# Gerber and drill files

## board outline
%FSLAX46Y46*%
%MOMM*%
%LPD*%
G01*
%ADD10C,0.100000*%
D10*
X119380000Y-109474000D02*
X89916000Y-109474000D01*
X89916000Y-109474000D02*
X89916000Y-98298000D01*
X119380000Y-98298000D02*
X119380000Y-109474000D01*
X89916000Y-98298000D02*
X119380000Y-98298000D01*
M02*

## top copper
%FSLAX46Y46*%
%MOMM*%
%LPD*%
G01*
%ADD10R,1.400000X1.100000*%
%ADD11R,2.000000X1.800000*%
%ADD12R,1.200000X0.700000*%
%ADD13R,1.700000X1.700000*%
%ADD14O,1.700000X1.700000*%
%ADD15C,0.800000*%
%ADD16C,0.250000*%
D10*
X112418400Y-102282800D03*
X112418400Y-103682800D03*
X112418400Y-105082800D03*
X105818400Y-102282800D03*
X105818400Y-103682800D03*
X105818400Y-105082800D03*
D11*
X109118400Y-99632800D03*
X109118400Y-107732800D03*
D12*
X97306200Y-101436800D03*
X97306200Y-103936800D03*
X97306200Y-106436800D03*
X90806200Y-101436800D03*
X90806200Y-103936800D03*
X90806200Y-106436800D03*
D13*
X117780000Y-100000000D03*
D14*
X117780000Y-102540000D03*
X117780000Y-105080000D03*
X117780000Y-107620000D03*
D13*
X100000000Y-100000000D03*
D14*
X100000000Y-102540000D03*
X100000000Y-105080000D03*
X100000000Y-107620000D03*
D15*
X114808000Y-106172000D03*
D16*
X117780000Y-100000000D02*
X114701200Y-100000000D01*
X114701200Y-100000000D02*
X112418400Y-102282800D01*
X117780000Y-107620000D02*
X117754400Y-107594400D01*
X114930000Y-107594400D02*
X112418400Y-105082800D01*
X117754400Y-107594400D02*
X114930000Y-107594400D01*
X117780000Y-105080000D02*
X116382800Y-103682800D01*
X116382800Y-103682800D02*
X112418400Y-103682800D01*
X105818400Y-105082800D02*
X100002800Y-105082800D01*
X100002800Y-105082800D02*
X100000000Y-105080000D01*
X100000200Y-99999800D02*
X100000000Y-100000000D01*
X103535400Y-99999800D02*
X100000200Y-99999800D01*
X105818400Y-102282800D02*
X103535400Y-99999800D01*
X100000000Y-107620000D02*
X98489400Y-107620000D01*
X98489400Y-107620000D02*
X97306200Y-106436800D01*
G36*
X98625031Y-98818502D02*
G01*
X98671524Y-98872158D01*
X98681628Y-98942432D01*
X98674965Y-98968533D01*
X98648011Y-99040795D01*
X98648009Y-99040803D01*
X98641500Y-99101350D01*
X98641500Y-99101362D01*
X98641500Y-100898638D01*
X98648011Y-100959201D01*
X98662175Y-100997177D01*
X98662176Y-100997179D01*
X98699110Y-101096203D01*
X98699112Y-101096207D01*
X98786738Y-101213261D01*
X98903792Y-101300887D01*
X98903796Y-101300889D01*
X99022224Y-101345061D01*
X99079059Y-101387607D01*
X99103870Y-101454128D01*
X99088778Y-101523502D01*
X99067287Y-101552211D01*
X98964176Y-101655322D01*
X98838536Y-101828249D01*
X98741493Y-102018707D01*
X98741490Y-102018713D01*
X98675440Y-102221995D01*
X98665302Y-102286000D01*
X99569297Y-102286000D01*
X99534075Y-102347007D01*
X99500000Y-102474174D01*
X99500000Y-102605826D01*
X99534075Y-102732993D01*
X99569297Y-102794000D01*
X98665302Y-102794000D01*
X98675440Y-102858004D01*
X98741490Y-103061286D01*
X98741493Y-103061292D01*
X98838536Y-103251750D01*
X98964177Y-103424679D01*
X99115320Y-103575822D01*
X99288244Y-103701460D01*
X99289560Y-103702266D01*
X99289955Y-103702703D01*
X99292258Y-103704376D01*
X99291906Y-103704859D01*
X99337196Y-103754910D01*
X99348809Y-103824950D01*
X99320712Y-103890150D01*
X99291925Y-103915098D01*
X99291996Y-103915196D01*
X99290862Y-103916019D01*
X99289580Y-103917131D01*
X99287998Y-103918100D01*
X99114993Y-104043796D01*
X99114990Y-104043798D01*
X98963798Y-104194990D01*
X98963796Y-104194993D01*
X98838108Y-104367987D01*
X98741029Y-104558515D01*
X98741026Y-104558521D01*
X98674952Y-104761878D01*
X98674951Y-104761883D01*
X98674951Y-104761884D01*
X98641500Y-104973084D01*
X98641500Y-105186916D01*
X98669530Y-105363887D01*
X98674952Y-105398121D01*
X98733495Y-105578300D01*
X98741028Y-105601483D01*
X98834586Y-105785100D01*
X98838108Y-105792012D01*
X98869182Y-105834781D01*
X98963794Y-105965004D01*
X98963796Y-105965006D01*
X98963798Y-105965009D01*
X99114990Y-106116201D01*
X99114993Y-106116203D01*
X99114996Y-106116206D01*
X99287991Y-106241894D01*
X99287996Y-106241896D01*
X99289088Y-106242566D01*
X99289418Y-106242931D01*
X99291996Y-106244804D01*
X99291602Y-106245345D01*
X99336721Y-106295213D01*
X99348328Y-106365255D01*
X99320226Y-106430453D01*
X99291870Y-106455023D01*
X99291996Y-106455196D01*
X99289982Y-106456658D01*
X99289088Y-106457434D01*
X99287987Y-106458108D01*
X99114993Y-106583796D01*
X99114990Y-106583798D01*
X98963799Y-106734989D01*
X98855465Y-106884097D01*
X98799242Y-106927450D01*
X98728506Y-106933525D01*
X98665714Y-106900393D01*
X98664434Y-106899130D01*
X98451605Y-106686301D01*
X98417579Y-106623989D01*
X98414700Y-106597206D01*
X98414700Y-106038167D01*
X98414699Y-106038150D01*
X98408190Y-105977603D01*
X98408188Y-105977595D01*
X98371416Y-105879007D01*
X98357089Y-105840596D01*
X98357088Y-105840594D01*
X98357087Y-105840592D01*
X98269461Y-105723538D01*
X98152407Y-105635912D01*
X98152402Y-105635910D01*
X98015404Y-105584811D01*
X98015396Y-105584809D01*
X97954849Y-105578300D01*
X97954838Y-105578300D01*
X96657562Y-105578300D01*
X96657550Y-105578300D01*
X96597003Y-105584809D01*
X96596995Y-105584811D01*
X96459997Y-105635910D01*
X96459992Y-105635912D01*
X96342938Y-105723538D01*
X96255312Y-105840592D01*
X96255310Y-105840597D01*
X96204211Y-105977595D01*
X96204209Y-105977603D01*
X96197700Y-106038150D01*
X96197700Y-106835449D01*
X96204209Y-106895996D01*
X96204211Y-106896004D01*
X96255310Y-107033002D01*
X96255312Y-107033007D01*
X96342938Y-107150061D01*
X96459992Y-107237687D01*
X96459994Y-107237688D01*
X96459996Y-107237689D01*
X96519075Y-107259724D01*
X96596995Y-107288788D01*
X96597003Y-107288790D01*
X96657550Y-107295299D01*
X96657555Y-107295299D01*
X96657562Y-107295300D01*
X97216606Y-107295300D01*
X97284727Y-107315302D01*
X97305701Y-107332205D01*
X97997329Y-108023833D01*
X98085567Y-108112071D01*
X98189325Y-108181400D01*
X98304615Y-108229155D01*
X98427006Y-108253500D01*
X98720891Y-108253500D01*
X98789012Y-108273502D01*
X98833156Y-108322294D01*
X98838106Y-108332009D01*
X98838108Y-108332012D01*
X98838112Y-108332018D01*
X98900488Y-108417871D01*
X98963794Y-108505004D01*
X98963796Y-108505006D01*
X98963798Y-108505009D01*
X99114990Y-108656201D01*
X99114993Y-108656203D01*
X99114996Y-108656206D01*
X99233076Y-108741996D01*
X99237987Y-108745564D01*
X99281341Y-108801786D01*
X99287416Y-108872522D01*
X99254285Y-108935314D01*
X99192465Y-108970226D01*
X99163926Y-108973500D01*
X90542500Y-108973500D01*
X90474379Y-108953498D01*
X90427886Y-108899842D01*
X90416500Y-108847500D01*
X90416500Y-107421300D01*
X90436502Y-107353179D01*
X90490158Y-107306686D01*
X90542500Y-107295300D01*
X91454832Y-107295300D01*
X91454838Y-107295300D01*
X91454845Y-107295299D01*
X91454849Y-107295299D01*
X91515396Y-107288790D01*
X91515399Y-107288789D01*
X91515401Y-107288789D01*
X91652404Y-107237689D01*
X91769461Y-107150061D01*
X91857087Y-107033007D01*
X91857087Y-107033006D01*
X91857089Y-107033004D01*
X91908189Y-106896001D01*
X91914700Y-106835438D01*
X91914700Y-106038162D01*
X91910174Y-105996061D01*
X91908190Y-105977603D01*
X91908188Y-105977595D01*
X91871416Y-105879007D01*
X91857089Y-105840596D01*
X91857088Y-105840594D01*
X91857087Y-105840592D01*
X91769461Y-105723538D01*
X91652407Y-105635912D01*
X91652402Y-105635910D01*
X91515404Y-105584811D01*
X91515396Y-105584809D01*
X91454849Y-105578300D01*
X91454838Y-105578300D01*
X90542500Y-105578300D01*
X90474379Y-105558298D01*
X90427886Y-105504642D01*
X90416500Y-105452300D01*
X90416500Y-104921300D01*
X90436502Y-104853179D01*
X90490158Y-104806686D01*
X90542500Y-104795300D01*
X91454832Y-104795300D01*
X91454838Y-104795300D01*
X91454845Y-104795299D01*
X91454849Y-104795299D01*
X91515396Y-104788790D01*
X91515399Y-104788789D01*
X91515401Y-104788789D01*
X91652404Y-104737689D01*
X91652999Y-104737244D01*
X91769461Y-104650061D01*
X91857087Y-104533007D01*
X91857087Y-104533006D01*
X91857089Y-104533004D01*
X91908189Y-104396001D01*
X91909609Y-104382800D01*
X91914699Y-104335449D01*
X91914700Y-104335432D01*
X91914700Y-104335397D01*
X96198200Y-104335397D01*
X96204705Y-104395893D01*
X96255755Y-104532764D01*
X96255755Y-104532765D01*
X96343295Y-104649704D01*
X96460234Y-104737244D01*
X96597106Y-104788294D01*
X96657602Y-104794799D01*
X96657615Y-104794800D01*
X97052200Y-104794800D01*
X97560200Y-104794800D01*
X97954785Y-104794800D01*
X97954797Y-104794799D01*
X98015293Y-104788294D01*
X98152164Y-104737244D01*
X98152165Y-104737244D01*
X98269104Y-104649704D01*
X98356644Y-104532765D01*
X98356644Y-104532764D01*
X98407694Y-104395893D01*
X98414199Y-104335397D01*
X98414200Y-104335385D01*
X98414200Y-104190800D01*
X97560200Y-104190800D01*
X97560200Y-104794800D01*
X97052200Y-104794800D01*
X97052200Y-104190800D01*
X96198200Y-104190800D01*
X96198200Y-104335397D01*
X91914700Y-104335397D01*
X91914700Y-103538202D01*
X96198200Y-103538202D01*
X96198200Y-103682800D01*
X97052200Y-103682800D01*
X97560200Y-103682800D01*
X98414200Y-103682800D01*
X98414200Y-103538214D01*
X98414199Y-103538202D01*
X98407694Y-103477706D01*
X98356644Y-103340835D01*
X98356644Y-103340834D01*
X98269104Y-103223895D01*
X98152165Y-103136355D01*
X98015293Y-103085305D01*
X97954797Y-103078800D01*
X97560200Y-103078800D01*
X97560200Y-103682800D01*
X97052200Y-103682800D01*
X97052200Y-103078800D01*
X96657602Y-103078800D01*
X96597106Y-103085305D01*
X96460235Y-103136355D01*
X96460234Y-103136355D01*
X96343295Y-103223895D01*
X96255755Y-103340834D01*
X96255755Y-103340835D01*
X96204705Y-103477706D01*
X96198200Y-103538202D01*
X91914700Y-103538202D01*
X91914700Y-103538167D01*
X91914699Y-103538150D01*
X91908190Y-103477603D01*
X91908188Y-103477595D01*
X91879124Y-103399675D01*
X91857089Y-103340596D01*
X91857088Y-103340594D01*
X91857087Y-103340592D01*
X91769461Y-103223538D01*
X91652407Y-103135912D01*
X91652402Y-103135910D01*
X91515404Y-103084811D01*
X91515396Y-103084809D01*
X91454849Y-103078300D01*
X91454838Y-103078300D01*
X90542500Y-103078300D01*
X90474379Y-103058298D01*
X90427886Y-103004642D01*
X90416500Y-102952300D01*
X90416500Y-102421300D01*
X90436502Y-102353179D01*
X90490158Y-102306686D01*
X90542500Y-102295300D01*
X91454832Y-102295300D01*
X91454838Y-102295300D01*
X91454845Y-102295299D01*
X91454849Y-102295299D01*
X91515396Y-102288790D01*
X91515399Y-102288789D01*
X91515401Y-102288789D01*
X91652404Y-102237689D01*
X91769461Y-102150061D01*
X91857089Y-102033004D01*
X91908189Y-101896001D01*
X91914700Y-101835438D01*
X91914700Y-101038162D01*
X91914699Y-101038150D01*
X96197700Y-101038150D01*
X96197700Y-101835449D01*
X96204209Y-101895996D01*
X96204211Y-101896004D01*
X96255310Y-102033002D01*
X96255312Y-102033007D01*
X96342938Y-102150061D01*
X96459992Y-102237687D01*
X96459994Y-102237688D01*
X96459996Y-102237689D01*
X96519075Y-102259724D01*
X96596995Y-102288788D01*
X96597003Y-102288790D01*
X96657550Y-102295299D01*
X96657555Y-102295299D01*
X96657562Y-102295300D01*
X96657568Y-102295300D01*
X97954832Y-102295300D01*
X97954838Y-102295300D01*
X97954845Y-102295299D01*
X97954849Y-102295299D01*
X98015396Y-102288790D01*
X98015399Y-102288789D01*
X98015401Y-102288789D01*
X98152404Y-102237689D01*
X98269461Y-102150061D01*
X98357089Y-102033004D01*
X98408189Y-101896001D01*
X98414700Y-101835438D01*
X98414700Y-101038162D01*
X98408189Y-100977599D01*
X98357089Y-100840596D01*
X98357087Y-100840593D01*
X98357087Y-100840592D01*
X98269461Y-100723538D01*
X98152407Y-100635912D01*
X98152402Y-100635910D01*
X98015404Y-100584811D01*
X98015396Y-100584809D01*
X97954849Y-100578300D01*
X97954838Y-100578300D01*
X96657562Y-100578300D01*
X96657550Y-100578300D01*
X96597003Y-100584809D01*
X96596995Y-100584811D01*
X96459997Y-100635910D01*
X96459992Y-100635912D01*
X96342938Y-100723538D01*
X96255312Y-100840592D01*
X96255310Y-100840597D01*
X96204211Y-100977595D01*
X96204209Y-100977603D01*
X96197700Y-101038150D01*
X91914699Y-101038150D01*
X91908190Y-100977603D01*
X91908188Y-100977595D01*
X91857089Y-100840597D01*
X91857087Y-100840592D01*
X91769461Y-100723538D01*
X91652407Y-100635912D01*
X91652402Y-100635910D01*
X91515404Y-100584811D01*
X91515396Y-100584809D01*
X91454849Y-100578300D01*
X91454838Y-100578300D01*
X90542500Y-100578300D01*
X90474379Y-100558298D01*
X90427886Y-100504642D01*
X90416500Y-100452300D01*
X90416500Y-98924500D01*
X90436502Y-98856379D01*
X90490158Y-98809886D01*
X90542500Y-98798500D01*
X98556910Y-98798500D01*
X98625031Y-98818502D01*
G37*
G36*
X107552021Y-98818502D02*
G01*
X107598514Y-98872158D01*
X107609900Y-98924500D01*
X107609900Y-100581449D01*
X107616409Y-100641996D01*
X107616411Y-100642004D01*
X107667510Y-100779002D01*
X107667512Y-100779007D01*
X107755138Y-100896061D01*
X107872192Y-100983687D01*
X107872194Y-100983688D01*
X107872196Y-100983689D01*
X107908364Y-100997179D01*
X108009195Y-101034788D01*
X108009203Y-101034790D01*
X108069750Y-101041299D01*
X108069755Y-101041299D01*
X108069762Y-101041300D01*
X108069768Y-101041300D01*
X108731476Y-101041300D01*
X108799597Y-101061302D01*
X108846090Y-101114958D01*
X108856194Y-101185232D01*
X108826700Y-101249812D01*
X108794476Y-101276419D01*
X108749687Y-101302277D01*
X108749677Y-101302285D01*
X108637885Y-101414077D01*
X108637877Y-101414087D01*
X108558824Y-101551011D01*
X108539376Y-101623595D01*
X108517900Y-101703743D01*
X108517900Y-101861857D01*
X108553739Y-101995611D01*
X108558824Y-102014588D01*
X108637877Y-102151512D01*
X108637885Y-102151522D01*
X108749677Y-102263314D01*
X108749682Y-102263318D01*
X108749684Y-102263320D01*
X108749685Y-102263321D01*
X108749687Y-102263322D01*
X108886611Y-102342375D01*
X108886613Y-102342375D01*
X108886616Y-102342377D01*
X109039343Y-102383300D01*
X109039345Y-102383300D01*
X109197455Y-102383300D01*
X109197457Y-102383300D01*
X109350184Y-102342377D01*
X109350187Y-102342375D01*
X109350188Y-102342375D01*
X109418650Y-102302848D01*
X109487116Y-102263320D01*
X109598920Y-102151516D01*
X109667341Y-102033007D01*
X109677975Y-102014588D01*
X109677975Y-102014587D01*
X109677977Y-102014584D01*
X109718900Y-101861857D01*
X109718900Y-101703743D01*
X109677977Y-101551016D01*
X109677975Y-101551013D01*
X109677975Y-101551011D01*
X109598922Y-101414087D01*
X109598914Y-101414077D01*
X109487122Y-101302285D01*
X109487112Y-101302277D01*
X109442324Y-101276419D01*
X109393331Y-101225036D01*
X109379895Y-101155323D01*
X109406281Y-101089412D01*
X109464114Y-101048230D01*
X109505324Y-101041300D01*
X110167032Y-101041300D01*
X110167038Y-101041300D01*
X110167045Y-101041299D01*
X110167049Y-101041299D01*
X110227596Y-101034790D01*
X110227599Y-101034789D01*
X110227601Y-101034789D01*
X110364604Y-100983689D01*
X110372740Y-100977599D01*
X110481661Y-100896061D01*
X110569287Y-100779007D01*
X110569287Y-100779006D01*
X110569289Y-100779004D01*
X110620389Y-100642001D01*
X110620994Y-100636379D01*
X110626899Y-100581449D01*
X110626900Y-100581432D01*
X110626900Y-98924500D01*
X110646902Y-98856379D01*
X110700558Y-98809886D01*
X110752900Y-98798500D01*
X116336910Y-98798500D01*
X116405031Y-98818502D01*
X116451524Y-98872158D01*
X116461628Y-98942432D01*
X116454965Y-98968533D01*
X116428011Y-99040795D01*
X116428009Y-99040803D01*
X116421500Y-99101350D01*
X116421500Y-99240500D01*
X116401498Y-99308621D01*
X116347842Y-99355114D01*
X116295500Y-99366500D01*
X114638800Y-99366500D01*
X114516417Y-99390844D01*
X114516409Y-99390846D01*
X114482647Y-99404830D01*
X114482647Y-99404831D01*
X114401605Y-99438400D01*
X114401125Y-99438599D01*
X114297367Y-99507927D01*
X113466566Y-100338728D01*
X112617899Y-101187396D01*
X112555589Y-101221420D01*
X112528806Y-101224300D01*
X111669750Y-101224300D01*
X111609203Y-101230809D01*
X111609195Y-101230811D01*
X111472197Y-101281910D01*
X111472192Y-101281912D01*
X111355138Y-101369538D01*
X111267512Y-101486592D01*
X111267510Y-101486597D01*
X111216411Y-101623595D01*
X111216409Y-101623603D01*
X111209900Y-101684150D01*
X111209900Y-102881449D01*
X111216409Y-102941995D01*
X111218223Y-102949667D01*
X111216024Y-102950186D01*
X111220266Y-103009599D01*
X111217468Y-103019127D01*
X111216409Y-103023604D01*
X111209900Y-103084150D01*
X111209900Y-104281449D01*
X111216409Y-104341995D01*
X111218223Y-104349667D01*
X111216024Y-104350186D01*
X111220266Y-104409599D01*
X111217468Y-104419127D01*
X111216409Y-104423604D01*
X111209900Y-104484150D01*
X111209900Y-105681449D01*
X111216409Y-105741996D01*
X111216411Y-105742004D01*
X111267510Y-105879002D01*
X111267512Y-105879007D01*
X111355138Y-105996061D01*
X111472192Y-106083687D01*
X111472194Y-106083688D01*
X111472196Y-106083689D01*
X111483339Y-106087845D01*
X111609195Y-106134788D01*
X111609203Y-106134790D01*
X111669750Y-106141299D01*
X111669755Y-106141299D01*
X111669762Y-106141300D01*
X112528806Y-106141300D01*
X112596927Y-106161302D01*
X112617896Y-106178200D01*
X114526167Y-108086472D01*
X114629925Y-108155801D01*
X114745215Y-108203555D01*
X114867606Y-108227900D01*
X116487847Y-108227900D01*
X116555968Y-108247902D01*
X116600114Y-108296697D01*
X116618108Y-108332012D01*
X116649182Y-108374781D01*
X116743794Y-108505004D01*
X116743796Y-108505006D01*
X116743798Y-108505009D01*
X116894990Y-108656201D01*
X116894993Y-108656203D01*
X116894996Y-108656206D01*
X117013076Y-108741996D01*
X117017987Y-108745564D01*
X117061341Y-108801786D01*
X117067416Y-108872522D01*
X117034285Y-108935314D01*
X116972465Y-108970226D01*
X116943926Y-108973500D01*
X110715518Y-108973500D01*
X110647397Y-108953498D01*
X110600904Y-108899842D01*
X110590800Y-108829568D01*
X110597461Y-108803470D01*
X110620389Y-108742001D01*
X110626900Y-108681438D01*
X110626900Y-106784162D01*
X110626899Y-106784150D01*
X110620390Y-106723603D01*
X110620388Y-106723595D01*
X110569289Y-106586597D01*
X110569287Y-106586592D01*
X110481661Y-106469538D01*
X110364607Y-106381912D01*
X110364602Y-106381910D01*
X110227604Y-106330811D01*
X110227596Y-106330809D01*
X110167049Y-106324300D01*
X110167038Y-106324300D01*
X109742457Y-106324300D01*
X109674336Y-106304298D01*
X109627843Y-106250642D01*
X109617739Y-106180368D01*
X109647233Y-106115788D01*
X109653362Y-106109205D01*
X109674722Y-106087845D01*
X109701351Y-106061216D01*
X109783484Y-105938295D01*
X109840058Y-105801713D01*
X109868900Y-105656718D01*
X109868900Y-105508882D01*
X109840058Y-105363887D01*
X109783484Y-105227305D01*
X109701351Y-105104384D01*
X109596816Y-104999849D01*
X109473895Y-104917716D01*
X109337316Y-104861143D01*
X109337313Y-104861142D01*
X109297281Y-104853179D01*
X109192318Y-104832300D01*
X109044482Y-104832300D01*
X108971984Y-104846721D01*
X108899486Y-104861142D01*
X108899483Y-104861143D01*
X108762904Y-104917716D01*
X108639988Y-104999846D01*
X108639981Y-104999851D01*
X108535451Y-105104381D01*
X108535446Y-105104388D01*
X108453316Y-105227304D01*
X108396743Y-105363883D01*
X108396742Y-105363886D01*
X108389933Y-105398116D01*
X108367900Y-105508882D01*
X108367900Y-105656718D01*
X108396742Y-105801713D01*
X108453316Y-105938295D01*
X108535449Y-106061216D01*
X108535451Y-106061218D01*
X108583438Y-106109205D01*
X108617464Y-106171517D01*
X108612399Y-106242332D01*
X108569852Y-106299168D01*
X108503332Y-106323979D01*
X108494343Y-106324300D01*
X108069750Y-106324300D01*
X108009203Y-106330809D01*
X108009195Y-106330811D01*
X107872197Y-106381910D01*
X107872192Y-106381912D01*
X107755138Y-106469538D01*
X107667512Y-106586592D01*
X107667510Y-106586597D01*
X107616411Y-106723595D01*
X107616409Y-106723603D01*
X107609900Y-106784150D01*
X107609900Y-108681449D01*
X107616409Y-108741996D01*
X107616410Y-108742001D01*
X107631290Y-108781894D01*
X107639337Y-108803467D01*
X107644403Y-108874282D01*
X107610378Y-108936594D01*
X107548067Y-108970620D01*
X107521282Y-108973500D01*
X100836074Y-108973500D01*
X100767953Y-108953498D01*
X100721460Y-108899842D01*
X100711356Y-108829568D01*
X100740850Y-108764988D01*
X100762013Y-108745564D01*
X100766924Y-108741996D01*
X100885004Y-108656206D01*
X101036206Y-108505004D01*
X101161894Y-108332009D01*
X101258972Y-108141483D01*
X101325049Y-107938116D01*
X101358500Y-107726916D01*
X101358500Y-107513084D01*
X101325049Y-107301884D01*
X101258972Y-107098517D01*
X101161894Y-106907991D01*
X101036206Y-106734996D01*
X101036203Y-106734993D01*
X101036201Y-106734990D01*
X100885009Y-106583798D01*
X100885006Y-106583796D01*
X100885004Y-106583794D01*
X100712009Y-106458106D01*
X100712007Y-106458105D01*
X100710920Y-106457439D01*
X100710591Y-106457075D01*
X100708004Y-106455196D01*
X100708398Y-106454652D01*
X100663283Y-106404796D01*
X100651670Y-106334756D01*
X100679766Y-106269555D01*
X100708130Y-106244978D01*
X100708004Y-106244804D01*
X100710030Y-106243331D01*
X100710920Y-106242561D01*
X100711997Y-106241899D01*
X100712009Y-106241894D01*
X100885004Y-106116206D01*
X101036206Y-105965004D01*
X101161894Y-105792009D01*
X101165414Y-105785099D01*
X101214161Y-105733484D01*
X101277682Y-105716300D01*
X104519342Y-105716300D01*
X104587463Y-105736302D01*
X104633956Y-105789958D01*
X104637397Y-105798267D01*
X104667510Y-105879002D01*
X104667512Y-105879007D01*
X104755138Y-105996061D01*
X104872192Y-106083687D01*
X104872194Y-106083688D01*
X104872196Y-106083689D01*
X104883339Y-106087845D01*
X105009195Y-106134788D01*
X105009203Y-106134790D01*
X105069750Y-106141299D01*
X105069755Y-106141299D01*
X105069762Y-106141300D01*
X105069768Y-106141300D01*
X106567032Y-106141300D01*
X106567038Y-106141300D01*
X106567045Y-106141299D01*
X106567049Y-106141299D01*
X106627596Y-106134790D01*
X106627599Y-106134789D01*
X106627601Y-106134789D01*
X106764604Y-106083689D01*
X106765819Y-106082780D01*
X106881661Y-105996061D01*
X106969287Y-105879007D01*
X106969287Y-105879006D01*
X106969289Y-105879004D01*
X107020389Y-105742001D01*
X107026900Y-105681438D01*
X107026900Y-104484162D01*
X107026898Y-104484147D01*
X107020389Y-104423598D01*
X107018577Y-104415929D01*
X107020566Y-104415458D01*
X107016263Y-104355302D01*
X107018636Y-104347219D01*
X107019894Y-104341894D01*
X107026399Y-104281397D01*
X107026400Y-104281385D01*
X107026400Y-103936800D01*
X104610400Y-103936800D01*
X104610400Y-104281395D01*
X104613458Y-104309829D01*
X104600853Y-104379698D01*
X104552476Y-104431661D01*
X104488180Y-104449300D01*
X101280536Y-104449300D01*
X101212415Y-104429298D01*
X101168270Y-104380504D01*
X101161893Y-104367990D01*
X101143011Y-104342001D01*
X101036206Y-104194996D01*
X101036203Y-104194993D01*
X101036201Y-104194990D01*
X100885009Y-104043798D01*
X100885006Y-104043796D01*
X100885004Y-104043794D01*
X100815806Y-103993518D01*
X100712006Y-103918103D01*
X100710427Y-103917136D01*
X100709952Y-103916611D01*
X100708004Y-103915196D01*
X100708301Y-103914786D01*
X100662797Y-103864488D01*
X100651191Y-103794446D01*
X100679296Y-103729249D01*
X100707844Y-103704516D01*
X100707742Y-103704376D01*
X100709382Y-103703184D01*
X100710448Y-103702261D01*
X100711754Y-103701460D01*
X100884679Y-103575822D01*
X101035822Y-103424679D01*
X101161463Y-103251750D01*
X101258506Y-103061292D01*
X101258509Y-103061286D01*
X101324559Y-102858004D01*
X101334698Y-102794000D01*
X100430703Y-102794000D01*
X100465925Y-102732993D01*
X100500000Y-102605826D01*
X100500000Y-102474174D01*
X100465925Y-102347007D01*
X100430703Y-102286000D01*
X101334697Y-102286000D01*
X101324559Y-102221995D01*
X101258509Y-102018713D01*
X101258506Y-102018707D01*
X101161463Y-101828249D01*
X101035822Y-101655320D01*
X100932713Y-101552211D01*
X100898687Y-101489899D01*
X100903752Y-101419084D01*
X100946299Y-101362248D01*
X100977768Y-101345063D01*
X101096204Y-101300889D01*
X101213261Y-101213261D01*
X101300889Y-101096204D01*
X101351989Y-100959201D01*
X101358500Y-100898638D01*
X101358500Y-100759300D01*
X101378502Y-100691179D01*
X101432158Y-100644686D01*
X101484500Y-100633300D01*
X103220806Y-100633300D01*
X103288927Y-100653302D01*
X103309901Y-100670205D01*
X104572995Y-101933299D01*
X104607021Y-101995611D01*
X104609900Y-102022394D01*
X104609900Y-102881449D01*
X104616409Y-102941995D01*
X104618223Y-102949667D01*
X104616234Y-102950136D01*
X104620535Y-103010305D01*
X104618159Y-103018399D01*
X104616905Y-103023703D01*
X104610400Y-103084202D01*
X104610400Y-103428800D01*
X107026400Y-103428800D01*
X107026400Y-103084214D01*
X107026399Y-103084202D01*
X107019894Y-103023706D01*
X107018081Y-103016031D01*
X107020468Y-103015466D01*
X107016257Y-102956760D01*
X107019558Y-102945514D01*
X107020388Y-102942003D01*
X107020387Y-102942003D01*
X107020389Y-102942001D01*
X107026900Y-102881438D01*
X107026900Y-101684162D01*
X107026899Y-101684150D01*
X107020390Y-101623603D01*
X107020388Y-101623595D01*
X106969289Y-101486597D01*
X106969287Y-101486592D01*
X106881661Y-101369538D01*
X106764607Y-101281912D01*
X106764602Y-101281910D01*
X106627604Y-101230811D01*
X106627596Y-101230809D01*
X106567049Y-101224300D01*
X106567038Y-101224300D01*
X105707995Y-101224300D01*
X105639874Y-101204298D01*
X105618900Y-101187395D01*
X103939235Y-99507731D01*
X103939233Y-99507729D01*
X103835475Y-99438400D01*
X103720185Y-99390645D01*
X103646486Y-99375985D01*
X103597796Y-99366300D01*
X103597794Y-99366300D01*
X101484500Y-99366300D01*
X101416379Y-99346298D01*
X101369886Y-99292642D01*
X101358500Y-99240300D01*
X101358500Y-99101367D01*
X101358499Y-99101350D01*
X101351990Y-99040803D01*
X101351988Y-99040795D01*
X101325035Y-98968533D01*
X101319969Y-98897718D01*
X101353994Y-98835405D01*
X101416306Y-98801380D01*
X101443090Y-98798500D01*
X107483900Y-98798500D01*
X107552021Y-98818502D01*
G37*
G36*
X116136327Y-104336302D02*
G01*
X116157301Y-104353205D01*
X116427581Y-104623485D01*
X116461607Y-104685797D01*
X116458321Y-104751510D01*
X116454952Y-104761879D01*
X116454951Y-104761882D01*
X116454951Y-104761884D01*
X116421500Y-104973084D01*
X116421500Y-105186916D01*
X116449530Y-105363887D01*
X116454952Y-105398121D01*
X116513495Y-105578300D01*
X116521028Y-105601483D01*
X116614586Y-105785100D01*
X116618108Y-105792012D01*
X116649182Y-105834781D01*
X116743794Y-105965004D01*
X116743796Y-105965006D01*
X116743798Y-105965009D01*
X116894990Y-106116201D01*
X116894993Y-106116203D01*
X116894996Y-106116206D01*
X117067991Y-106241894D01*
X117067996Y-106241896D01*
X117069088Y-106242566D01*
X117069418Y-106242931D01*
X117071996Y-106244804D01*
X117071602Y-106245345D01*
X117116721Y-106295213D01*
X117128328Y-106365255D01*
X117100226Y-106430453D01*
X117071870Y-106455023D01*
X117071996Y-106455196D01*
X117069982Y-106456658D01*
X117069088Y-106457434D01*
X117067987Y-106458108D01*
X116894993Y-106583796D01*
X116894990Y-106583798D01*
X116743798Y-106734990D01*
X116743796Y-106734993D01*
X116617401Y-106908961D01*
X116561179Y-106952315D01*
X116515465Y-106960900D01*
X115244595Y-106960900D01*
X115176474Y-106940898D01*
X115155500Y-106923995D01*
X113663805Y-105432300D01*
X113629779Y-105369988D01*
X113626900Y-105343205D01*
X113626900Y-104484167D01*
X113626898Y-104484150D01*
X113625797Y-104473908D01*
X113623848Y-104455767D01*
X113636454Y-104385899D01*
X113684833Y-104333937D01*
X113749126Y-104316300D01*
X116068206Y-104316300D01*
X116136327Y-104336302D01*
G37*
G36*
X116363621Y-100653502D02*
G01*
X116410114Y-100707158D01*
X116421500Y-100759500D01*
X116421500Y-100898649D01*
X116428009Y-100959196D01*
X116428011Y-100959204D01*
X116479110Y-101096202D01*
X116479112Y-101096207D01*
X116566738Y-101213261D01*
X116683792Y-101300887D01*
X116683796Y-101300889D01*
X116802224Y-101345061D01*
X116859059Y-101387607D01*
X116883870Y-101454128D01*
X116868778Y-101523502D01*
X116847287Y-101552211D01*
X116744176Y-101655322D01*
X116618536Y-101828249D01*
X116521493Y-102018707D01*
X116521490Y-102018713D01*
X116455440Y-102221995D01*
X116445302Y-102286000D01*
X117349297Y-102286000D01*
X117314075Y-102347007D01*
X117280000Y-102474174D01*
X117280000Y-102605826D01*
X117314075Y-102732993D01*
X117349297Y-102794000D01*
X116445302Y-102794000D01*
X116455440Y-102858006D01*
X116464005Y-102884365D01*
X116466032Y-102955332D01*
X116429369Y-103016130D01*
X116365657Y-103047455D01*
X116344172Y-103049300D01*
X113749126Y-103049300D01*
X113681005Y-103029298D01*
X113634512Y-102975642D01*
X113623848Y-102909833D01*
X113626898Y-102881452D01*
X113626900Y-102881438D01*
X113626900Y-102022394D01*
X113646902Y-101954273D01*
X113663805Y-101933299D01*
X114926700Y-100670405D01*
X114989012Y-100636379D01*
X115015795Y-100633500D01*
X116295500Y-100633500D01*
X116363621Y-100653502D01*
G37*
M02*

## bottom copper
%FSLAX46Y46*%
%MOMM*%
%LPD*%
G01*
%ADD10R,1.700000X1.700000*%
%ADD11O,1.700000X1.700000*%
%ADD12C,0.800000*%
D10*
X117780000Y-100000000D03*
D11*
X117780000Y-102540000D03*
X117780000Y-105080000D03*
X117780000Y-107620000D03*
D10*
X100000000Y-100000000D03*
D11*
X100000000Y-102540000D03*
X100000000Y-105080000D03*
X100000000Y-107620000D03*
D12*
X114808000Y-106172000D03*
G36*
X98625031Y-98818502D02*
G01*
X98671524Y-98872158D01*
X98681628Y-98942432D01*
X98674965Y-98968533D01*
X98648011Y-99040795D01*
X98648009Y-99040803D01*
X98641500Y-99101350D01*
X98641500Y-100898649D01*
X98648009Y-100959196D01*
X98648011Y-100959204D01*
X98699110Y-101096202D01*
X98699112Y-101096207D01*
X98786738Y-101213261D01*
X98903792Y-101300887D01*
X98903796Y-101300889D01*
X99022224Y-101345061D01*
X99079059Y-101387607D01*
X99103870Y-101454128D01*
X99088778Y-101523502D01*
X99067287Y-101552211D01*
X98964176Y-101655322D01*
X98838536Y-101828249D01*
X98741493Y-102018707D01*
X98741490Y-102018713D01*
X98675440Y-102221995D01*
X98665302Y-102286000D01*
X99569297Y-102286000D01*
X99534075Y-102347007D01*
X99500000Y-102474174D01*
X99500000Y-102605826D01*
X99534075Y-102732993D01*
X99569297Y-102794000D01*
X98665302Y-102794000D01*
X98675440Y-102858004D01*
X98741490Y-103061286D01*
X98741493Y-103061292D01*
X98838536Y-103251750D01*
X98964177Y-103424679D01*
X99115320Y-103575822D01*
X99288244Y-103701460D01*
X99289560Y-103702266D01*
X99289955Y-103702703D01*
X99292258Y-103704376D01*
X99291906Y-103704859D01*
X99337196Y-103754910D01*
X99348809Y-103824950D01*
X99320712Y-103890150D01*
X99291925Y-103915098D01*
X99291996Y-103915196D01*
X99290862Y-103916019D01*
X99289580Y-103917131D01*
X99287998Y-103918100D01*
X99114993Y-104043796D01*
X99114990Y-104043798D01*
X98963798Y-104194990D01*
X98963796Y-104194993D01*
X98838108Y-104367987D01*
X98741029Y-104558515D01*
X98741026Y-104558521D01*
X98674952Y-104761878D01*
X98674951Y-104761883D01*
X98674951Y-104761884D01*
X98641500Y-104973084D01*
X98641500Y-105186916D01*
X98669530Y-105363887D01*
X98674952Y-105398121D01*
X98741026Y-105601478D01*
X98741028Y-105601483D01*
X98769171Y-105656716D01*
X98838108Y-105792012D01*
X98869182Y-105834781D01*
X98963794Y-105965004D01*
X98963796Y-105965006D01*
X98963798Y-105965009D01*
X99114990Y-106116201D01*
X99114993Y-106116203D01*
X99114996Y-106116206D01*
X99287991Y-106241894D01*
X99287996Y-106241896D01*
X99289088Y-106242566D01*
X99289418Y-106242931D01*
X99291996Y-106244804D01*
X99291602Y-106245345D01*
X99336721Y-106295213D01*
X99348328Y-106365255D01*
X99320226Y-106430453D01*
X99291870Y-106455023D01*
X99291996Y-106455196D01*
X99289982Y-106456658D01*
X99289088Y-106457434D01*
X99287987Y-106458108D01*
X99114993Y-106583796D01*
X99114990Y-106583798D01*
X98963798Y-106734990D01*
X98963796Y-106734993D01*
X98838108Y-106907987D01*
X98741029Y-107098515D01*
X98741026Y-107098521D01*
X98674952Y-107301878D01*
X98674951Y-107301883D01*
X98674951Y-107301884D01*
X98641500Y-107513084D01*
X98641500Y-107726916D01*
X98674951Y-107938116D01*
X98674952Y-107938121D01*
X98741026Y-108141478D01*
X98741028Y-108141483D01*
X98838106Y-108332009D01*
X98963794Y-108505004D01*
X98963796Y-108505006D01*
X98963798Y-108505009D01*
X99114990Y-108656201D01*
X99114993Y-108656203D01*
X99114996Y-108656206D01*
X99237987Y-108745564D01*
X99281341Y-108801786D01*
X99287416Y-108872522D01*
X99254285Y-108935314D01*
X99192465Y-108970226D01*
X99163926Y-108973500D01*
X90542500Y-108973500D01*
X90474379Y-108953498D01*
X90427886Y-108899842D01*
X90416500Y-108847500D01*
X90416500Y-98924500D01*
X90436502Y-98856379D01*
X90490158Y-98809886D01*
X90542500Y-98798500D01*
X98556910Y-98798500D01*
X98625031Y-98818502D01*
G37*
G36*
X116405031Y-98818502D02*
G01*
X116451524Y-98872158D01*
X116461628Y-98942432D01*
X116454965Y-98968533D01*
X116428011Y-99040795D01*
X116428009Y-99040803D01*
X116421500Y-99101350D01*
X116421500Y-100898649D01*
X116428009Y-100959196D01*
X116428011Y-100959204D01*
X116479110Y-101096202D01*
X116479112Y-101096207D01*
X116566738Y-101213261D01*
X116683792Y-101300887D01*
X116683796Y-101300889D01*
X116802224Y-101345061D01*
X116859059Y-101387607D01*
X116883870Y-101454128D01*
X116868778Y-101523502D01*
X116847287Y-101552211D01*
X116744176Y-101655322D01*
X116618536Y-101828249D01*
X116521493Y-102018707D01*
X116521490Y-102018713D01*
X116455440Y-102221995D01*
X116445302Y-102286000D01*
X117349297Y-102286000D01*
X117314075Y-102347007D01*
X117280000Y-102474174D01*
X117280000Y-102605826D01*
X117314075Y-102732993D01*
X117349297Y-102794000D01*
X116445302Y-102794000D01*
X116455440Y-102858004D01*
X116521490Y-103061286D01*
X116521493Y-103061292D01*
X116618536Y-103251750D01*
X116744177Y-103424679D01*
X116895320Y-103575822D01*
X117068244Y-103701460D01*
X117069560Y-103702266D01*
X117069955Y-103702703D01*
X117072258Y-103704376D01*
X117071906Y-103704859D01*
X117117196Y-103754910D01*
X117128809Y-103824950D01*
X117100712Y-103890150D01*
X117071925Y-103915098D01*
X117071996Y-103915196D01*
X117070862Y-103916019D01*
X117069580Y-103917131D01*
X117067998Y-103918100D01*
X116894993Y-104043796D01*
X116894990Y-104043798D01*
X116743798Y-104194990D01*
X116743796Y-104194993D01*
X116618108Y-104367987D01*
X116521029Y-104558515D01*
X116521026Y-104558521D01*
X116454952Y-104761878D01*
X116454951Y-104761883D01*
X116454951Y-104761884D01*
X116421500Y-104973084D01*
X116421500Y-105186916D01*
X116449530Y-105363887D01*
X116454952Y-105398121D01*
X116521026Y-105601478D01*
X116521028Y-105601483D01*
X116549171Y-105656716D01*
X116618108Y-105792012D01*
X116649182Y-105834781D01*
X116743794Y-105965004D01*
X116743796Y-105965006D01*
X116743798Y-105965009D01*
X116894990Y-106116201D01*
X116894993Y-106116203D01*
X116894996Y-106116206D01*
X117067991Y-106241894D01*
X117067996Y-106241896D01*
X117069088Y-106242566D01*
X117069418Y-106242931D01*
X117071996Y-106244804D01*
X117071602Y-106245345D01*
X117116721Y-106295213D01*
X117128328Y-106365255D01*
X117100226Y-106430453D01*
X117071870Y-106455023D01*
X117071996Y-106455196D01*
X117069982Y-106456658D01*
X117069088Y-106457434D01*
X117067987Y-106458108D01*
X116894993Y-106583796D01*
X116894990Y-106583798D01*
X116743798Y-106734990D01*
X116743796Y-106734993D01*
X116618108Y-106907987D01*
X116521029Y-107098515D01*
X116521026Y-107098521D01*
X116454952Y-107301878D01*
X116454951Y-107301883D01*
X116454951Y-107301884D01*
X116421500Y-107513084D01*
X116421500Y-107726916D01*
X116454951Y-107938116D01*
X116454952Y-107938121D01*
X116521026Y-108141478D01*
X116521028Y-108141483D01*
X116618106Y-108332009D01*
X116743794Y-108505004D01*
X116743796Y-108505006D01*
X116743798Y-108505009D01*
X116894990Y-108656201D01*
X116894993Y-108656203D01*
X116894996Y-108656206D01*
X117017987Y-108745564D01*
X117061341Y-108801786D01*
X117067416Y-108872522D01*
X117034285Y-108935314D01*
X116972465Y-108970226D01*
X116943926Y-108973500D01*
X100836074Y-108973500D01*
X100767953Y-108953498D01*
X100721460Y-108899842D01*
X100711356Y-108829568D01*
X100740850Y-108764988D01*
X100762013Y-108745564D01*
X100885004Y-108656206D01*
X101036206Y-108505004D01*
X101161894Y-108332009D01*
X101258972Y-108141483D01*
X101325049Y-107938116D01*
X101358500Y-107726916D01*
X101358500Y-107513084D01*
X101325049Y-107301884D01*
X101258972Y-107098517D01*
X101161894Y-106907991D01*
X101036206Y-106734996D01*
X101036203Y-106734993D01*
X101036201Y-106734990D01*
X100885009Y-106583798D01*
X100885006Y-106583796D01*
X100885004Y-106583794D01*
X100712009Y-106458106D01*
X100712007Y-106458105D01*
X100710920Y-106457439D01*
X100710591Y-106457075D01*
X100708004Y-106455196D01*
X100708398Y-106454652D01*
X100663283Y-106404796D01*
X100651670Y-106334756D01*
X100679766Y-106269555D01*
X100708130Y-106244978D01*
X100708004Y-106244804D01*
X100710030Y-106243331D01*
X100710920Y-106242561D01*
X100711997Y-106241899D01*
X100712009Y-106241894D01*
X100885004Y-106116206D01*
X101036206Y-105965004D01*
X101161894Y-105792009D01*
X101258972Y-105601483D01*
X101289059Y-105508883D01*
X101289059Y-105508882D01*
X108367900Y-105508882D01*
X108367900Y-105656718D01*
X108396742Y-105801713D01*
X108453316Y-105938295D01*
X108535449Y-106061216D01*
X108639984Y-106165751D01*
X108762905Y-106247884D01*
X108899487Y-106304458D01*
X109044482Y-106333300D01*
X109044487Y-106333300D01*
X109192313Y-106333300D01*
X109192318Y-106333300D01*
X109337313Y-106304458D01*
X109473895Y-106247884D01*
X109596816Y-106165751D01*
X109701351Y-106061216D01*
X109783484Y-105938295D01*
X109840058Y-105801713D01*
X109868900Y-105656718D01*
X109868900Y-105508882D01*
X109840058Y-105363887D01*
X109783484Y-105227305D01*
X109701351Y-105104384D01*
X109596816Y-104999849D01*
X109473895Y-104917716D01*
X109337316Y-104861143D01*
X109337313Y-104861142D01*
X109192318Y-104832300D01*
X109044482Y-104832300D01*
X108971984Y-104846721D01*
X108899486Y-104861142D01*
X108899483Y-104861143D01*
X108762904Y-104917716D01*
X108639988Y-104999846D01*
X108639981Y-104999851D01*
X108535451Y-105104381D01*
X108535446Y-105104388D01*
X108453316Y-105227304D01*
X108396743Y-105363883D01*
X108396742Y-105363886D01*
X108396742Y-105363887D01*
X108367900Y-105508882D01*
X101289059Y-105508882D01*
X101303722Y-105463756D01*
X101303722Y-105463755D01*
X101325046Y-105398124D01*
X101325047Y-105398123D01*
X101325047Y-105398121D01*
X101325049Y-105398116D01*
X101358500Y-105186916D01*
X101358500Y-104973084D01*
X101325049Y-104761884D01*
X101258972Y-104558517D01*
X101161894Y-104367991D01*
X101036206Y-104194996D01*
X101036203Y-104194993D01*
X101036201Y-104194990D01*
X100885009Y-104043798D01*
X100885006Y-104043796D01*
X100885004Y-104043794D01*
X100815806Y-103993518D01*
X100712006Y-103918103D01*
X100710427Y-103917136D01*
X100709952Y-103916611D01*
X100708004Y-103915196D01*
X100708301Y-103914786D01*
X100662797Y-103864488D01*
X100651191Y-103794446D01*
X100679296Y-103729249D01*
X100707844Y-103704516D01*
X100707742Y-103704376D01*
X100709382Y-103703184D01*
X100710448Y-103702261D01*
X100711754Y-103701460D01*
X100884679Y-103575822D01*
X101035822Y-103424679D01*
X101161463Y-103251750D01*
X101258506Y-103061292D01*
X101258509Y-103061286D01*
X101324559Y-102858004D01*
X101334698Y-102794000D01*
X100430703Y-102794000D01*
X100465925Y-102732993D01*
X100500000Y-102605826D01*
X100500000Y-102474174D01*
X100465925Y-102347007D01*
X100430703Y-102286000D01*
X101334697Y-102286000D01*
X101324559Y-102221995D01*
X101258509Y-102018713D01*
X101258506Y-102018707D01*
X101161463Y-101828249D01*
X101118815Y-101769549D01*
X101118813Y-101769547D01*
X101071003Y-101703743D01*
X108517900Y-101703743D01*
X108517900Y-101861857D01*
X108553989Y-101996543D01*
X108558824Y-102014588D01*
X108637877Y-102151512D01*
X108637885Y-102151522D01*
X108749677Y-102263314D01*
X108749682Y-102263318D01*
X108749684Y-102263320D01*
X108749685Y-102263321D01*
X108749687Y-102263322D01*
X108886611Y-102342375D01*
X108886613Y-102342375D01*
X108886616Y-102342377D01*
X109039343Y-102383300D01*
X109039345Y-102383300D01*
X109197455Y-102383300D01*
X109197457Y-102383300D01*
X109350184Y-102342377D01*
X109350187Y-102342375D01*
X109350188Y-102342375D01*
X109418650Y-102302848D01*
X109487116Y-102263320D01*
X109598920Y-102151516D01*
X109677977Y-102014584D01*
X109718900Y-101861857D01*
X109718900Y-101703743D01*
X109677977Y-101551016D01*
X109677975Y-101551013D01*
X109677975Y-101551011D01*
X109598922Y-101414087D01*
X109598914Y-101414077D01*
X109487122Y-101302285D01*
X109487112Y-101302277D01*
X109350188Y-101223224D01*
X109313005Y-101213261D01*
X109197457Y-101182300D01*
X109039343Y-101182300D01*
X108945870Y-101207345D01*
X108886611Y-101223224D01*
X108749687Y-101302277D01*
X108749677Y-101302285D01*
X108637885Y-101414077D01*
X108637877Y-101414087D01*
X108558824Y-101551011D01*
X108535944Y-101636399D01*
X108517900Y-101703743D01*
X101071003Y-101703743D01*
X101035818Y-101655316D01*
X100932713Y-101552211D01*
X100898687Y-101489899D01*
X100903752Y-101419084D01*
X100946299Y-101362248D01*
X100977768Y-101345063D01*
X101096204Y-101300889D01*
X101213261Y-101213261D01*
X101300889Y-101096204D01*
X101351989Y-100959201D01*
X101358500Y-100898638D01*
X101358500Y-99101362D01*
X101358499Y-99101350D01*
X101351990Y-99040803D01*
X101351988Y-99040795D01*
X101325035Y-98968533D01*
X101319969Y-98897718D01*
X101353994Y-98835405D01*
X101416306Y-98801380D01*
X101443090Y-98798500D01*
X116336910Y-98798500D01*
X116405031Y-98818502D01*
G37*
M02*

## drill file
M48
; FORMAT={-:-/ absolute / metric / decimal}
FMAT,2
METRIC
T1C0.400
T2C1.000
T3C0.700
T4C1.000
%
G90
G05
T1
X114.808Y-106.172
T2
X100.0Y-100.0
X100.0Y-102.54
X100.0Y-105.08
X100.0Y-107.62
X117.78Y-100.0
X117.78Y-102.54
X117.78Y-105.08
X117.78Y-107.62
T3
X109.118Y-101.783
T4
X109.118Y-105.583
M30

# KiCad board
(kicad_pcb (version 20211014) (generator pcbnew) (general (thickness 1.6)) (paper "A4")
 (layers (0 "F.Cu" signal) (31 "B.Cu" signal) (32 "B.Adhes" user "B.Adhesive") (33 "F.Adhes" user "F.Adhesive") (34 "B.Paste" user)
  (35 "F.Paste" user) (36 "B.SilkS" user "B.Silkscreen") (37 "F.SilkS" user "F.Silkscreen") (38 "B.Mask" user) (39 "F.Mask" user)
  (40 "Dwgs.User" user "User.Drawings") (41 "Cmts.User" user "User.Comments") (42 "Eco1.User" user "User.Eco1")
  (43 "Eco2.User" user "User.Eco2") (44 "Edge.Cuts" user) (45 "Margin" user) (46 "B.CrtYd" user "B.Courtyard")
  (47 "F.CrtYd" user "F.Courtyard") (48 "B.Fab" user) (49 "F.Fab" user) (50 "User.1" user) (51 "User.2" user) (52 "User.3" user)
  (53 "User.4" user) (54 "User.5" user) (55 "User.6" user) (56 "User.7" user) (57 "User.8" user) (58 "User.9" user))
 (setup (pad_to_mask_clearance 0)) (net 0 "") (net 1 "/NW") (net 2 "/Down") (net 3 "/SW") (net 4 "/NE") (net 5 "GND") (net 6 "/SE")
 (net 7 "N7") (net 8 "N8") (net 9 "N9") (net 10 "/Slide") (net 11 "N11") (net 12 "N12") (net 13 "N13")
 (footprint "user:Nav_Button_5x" (layer "F.Cu") (at 109.1184 103.6828 180)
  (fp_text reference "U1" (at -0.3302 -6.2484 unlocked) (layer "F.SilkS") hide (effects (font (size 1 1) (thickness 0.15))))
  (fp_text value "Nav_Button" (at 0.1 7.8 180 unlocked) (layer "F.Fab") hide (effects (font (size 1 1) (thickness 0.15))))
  (pad "" np_thru_hole circle (at 0 -1.9 180) (size 1 1) (drill 1) (layers *.Mask))
  (pad "" np_thru_hole circle (at 0 1.9 180) (size 0.7 0.7) (drill 0.7) (layers *.Mask))
  (pad "1" smd rect (at -3.3 1.4 180) (size 1.4 1.1) (layers "F.Cu" "F.Paste" "F.Mask") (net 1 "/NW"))
  (pad "2" smd rect (at -3.3 0 180) (size 1.4 1.1) (layers "F.Cu" "F.Paste" "F.Mask") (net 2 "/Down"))
  (pad "3" smd rect (at -3.3 -1.4 180) (size 1.4 1.1) (layers "F.Cu" "F.Paste" "F.Mask") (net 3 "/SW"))
  (pad "4" smd rect (at 3.3 1.4 180) (size 1.4 1.1) (layers "F.Cu" "F.Paste" "F.Mask") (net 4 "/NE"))
  (pad "5" smd rect (at 3.3 0 180) (size 1.4 1.1) (layers "F.Cu" "F.Paste" "F.Mask") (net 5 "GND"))
  (pad "6" smd rect (at 3.3 -1.4 180) (size 1.4 1.1) (layers "F.Cu" "F.Paste" "F.Mask") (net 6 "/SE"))
  (pad "7" smd rect (at 0 4.05 180) (size 2 1.8) (layers "F.Cu" "F.Paste" "F.Mask") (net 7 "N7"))
  (pad "8" smd rect (at 0 -4.05 180) (size 2 1.8) (layers "F.Cu" "F.Paste" "F.Mask") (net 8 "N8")))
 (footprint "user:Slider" (layer "F.Cu") (at 94.0562 103.9368 -90)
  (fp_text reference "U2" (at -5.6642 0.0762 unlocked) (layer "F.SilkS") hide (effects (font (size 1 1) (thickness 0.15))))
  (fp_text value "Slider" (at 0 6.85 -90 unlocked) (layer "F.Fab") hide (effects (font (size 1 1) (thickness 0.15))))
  (pad "1" smd rect (at -2.5 -3.25 270) (size 0.7 1.2) (layers "F.Cu" "F.Paste" "F.Mask") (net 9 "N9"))
  (pad "2" smd rect (at 0 -3.25 270) (size 0.7 1.2) (layers "F.Cu" "F.Paste" "F.Mask") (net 5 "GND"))
  (pad "3" smd rect (at 2.5 -3.25 270) (size 0.7 1.2) (layers "F.Cu" "F.Paste" "F.Mask") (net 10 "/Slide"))
  (pad "4" smd rect (at -2.5 3.25 270) (size 0.7 1.2) (layers "F.Cu" "F.Paste" "F.Mask") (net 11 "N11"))
  (pad "5" smd rect (at 0 3.25 270) (size 0.7 1.2) (layers "F.Cu" "F.Paste" "F.Mask") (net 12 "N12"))
  (pad "6" smd rect (at 2.5 3.25 270) (size 0.7 1.2) (layers "F.Cu" "F.Paste" "F.Mask") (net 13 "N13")))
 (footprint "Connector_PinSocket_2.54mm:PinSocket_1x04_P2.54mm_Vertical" (layer "B.Cu") (at 117.78 100 180)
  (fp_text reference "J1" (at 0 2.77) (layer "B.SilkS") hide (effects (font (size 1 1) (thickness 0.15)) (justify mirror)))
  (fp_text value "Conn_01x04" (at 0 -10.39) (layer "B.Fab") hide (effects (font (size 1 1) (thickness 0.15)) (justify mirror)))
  (pad "1" thru_hole rect (at 0 0 180) (size 1.7 1.7) (drill 1) (layers *.Cu *.Mask) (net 1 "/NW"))
  (pad "2" thru_hole oval (at 0 -2.54 180) (size 1.7 1.7) (drill 1) (layers *.Cu *.Mask) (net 5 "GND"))
  (pad "3" thru_hole oval (at 0 -5.08 180) (size 1.7 1.7) (drill 1) (layers *.Cu *.Mask) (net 2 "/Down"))
  (pad "4" thru_hole oval (at 0 -7.62 180) (size 1.7 1.7) (drill 1) (layers *.Cu *.Mask) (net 3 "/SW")))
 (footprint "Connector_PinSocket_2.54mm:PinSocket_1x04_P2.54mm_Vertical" (layer "B.Cu") (at 100 100 180)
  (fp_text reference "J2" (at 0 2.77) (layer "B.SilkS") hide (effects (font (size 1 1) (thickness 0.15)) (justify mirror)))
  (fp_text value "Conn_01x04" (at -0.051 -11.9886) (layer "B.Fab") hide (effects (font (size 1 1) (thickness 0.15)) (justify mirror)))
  (pad "1" thru_hole rect (at 0 0 180) (size 1.7 1.7) (drill 1) (layers *.Cu *.Mask) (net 4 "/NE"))
  (pad "2" thru_hole oval (at 0 -2.54 180) (size 1.7 1.7) (drill 1) (layers *.Cu *.Mask) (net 5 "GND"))
  (pad "3" thru_hole oval (at 0 -5.08 180) (size 1.7 1.7) (drill 1) (layers *.Cu *.Mask) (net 6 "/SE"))
  (pad "4" thru_hole oval (at 0 -7.62 180) (size 1.7 1.7) (drill 1) (layers *.Cu *.Mask) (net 10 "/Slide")))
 (gr_line (start 119.38 109.474) (end 89.916 109.474) (layer "Edge.Cuts") (width 0.1))
 (gr_line (start 89.916 109.474) (end 89.916 98.298) (layer "Edge.Cuts") (width 0.1))
 (gr_line (start 119.38 98.298) (end 119.38 109.474) (layer "Edge.Cuts") (width 0.1))
 (gr_line (start 89.916 98.298) (end 119.38 98.298) (layer "Edge.Cuts") (width 0.1))
 (segment (start 117.78 100) (end 114.7012 100) (width 0.25) (layer "F.Cu") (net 1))
 (segment (start 114.7012 100) (end 112.4184 102.2828) (width 0.25) (layer "F.Cu") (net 1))
 (via (at 114.808 106.172) (size 0.8) (drill 0.4) (layers "F.Cu" "B.Cu") (free) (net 5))
 (segment (start 117.78 107.62) (end 117.7544 107.5944) (width 0.25) (layer "F.Cu") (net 3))
 (segment (start 114.93 107.5944) (end 112.4184 105.0828) (width 0.25) (layer "F.Cu") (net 3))
 (segment (start 117.7544 107.5944) (end 114.93 107.5944) (width 0.25) (layer "F.Cu") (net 3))
 (segment (start 117.78 105.08) (end 116.3828 103.6828) (width 0.25) (layer "F.Cu") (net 2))
 (segment (start 116.3828 103.6828) (end 112.4184 103.6828) (width 0.25) (layer "F.Cu") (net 2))
 (segment (start 105.8184 105.0828) (end 100.0028 105.0828) (width 0.25) (layer "F.Cu") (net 6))
 (segment (start 100.0028 105.0828) (end 100 105.08) (width 0.25) (layer "F.Cu") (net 6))
 (segment (start 100.0002 99.9998) (end 100 100) (width 0.25) (layer "F.Cu") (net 4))
 (segment (start 103.5354 99.9998) (end 100.0002 99.9998) (width 0.25) (layer "F.Cu") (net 4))
 (segment (start 105.8184 102.2828) (end 103.5354 99.9998) (width 0.25) (layer "F.Cu") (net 4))
 (segment (start 100 107.62) (end 98.4894 107.62) (width 0.25) (layer "F.Cu") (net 10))
 (segment (start 98.4894 107.62) (end 97.3062 106.4368) (width 0.25) (layer "F.Cu") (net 10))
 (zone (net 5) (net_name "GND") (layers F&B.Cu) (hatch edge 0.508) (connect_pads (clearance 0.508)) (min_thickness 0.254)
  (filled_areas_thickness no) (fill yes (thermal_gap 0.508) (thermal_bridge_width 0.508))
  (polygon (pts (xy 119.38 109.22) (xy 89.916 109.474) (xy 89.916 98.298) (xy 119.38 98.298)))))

